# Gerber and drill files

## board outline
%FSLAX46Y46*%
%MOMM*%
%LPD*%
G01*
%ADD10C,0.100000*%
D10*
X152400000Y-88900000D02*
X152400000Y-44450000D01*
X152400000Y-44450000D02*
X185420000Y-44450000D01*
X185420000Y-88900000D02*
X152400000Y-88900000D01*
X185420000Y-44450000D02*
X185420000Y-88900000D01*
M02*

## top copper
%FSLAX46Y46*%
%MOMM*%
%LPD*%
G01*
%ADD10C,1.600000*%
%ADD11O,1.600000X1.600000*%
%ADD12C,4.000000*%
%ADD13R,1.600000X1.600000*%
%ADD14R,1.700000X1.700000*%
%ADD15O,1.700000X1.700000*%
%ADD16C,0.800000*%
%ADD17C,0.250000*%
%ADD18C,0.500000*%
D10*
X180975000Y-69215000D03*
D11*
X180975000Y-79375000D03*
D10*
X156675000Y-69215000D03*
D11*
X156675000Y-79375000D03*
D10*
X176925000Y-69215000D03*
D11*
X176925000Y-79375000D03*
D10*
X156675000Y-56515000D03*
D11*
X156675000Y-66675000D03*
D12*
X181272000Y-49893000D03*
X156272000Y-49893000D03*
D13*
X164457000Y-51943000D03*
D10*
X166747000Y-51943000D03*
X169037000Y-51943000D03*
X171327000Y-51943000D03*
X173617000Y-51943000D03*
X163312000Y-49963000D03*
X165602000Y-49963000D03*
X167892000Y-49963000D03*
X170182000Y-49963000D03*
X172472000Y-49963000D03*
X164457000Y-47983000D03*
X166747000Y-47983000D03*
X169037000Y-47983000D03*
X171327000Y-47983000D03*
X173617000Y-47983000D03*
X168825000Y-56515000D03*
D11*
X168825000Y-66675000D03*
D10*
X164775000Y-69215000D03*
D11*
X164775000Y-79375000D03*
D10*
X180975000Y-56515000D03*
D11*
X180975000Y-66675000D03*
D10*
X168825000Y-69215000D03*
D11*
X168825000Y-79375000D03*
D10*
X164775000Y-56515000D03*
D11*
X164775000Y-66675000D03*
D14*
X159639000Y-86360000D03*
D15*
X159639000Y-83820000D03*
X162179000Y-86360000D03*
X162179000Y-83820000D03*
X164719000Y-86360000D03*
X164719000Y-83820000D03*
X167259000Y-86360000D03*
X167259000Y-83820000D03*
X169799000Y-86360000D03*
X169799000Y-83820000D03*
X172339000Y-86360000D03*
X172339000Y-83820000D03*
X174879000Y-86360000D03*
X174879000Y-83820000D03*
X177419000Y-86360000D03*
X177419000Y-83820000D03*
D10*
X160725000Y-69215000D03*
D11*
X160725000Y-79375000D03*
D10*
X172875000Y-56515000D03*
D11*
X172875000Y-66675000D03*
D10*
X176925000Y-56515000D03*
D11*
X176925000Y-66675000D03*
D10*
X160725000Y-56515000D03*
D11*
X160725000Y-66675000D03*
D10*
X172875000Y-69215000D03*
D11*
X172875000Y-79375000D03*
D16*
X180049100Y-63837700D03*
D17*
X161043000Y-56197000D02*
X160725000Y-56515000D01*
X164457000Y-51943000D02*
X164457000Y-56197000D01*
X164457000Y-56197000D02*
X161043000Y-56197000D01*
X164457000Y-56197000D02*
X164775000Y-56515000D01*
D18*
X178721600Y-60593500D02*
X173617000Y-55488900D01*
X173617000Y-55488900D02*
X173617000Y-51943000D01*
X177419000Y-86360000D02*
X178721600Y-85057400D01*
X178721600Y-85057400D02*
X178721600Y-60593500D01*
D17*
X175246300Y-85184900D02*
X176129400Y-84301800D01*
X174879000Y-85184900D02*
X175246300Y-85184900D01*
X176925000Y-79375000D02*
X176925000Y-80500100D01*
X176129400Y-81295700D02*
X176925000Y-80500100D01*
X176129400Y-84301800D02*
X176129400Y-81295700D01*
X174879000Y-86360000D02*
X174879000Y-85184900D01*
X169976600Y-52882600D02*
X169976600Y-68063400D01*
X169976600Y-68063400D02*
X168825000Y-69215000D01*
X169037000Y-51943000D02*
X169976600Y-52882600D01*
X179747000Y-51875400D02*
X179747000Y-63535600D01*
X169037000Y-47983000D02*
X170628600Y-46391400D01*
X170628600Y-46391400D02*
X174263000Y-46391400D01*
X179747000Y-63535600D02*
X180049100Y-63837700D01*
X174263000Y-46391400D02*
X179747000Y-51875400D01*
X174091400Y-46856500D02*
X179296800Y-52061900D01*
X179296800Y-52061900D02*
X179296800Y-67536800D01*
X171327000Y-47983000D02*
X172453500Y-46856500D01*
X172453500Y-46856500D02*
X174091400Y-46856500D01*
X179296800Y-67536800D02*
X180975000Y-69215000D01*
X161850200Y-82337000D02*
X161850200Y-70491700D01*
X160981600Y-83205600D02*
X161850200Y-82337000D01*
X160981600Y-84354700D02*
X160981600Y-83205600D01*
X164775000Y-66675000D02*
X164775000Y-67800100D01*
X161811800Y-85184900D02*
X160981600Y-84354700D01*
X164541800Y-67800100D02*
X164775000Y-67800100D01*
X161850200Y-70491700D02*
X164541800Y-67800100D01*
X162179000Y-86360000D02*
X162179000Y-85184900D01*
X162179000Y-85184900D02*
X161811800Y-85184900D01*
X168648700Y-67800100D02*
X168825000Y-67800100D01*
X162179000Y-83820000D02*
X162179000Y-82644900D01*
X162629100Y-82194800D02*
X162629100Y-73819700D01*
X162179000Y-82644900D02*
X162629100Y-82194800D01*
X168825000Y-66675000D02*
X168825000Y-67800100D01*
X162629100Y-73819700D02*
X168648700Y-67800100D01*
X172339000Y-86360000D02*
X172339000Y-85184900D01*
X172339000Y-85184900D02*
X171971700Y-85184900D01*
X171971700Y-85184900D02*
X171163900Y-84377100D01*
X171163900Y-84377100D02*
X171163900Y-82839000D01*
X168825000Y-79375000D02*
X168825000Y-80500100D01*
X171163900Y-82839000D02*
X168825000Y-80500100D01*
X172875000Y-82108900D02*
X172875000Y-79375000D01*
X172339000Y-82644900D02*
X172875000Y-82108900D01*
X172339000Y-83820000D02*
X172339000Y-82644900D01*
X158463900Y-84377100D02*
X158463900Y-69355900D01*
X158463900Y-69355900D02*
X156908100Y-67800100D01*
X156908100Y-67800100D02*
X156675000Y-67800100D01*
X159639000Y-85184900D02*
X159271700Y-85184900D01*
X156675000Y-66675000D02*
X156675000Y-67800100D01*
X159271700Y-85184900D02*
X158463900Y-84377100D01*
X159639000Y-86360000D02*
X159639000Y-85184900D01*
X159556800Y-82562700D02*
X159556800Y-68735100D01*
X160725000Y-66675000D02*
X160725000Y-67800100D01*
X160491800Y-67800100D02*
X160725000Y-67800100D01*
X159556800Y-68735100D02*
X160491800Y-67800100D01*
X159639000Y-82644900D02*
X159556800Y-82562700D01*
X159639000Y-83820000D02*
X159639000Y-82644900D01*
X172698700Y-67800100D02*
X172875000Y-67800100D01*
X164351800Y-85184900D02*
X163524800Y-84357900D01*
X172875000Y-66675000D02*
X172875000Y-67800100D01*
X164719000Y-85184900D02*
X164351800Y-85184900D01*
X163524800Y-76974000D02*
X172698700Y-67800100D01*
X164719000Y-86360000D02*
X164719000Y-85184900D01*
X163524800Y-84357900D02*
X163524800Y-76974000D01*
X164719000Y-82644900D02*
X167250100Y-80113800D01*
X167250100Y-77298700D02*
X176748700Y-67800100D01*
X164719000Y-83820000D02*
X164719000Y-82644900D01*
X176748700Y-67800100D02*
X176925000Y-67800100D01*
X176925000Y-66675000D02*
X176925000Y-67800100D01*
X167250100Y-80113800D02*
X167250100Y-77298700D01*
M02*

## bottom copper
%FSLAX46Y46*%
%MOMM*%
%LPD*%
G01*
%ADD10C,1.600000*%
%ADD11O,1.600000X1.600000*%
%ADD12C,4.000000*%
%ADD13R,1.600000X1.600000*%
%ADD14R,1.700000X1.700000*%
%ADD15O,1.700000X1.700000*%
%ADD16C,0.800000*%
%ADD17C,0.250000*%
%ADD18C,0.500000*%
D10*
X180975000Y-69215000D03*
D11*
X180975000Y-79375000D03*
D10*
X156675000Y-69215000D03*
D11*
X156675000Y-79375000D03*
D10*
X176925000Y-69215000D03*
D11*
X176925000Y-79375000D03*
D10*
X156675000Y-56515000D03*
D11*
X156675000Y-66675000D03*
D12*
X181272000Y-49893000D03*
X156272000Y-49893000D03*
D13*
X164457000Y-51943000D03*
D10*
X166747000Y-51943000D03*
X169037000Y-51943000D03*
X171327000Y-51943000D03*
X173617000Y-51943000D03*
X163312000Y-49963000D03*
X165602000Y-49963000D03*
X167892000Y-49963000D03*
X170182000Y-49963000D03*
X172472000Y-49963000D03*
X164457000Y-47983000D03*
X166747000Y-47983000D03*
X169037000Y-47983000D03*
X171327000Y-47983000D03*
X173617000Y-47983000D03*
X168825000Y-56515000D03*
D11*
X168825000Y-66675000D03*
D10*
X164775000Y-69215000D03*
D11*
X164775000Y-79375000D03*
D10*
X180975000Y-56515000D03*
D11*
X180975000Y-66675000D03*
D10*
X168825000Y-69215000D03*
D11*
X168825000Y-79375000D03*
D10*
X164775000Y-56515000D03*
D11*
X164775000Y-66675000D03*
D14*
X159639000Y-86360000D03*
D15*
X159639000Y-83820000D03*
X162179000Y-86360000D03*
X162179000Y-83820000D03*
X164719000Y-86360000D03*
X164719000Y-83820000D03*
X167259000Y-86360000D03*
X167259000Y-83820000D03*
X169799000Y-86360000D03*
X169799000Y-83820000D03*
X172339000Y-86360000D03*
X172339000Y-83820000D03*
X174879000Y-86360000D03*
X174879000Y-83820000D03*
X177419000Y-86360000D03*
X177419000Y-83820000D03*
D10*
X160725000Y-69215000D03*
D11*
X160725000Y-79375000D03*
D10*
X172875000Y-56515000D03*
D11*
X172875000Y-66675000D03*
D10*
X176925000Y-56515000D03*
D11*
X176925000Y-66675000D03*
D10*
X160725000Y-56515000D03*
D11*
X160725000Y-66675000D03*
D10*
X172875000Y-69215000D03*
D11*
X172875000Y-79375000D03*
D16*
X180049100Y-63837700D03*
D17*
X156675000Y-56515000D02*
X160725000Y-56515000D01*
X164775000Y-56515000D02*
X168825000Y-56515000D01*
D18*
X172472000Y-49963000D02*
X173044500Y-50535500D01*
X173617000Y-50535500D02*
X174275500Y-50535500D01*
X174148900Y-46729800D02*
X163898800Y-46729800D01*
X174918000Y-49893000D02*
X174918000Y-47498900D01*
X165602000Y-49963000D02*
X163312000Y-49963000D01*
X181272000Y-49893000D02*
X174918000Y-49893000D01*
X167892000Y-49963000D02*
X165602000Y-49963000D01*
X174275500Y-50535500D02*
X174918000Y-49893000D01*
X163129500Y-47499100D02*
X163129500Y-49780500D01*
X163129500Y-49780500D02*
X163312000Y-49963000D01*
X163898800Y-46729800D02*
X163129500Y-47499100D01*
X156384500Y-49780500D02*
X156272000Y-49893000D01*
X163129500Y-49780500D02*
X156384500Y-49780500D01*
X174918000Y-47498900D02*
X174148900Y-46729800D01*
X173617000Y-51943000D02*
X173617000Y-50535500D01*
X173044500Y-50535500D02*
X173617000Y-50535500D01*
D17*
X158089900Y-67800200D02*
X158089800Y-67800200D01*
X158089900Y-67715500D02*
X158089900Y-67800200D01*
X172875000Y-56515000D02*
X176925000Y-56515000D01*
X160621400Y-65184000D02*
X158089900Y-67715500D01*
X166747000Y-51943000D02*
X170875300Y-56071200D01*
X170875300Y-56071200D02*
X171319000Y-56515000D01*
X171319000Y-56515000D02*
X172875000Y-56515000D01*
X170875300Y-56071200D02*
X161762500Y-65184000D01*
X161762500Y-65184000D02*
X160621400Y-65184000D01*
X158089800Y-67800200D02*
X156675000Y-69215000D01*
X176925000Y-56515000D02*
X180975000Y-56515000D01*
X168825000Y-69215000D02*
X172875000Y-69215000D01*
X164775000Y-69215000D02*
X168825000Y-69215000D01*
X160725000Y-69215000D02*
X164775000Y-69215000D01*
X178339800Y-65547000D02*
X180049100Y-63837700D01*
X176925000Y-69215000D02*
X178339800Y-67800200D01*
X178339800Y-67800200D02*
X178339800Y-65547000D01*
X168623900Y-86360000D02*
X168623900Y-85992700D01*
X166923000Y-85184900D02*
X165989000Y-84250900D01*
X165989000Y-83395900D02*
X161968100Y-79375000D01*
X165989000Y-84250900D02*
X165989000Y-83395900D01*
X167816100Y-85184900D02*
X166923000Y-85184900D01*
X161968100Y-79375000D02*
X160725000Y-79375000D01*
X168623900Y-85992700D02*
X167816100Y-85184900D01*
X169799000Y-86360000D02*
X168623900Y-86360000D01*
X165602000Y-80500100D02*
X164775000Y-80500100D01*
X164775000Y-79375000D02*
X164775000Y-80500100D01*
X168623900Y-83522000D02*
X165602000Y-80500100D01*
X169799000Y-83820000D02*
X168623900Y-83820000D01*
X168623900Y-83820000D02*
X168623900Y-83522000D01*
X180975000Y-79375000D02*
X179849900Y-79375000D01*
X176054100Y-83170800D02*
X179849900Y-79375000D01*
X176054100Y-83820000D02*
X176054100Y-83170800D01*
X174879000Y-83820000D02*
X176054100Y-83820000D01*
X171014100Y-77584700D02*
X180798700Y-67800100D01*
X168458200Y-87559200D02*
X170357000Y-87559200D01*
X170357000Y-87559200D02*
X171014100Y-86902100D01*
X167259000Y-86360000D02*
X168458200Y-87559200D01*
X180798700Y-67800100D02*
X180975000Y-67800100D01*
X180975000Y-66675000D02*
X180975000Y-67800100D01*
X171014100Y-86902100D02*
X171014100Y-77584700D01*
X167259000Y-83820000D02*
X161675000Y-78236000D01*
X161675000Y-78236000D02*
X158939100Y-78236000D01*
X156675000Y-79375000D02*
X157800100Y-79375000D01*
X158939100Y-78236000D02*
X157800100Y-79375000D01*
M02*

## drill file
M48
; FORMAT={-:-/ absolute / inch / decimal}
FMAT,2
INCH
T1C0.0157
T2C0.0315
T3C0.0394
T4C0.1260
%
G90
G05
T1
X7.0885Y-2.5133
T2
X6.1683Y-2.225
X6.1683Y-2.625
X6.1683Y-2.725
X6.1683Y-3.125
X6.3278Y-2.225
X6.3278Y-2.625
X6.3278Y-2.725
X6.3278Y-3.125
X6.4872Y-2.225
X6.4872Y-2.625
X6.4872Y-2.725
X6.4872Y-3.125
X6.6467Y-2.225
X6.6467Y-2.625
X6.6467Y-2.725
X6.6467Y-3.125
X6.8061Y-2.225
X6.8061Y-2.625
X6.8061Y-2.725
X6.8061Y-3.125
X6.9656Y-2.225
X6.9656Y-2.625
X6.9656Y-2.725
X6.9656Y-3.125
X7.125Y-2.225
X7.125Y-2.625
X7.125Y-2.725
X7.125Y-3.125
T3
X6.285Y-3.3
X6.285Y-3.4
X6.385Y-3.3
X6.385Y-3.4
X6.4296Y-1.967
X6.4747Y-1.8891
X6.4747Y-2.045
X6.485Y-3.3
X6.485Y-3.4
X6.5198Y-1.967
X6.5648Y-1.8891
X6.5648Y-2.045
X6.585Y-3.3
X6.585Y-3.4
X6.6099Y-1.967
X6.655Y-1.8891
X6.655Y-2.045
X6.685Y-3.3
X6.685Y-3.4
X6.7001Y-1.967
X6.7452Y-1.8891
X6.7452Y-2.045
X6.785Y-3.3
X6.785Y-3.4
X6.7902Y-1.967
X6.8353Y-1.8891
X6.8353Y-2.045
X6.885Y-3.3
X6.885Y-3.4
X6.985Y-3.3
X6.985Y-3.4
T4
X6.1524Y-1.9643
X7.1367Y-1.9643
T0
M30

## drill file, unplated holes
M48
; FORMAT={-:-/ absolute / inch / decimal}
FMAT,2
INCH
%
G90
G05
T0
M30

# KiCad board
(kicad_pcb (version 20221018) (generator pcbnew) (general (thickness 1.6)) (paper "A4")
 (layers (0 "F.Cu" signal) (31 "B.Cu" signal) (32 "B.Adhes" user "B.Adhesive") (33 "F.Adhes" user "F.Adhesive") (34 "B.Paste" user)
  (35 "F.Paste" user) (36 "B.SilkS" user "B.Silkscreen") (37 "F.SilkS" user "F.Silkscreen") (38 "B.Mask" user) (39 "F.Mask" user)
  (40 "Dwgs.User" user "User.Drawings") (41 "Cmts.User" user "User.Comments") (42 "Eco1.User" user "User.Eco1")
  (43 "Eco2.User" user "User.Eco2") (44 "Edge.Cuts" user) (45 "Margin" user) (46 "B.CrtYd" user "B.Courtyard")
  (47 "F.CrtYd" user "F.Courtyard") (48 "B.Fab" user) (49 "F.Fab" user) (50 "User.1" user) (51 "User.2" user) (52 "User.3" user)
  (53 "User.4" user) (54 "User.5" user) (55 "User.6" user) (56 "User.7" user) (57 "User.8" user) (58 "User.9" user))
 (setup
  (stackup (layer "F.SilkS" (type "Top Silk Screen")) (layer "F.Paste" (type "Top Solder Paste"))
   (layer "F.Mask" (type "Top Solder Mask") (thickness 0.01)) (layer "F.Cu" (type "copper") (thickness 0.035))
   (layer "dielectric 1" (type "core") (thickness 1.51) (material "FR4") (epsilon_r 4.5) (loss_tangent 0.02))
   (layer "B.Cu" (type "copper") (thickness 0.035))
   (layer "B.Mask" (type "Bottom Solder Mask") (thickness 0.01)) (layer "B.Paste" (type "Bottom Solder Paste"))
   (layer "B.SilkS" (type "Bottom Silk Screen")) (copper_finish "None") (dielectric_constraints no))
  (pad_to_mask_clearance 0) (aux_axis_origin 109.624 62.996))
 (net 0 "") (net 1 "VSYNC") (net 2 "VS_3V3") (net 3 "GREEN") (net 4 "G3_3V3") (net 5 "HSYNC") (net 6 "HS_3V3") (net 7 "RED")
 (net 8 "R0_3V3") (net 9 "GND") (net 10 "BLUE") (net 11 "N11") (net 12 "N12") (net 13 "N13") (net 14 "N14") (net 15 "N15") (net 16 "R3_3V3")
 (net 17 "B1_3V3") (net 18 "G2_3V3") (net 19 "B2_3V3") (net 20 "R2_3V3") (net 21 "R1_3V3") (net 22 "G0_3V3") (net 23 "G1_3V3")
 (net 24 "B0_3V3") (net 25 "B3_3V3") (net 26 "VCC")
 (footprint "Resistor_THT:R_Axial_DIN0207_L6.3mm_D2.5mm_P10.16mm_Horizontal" (layer "F.Cu") (at 180.975 69.215 -90)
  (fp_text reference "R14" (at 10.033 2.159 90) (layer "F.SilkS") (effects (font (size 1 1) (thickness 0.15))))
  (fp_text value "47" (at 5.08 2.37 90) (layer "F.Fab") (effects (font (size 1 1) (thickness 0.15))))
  (pad "1" thru_hole circle (at 0 0 270) (size 1.6 1.6) (drill 0.8) (layers "*.Cu" "*.Mask") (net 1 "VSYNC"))
  (pad "2" thru_hole oval (at 10.16 0 270) (size 1.6 1.6) (drill 0.8) (layers "*.Cu" "*.Mask") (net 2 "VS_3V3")))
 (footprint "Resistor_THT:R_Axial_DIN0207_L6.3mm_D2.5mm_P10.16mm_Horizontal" (layer "F.Cu") (at 156.675 69.215 -90)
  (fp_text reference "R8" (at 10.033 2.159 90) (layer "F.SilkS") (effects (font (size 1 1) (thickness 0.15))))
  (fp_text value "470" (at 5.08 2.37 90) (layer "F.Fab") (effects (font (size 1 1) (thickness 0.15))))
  (pad "1" thru_hole circle (at 0 0 270) (size 1.6 1.6) (drill 0.8) (layers "*.Cu" "*.Mask") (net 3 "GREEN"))
  (pad "2" thru_hole oval (at 10.16 0 270) (size 1.6 1.6) (drill 0.8) (layers "*.Cu" "*.Mask") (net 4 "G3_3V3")))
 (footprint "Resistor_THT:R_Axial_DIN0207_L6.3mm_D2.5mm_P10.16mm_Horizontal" (layer "F.Cu") (at 176.925 69.215 -90)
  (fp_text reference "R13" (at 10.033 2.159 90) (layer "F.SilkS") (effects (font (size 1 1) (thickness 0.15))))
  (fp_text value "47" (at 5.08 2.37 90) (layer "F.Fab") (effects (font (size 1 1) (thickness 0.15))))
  (pad "1" thru_hole circle (at 0 0 270) (size 1.6 1.6) (drill 0.8) (layers "*.Cu" "*.Mask") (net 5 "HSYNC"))
  (pad "2" thru_hole oval (at 10.16 0 270) (size 1.6 1.6) (drill 0.8) (layers "*.Cu" "*.Mask") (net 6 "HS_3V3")))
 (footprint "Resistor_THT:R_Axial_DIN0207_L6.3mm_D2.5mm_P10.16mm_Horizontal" (layer "F.Cu") (at 156.675 56.515 -90)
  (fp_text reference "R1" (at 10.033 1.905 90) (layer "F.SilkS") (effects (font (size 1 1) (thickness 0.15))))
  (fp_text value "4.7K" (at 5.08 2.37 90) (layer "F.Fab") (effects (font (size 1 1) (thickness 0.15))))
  (pad "1" thru_hole circle (at 0 0 270) (size 1.6 1.6) (drill 0.8) (layers "*.Cu" "*.Mask") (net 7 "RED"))
  (pad "2" thru_hole oval (at 10.16 0 270) (size 1.6 1.6) (drill 0.8) (layers "*.Cu" "*.Mask") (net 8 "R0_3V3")))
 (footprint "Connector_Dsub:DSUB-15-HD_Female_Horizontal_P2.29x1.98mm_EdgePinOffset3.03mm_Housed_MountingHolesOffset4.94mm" (layer "F.Cu")
  (at 164.457 51.943 180)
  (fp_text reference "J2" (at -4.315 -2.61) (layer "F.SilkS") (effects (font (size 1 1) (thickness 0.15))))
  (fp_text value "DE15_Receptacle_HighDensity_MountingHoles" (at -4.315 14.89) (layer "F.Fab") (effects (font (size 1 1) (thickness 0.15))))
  (pad "0" thru_hole circle (at -16.815 2.05 180) (size 4 4) (drill 3.2) (layers "*.Cu" "*.Mask") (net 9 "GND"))
  (pad "0" thru_hole circle (at 8.185 2.05 180) (size 4 4) (drill 3.2) (layers "*.Cu" "*.Mask") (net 9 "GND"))
  (pad "1" thru_hole rect (at 0 0 180) (size 1.6 1.6) (drill 1) (layers "*.Cu" "*.Mask") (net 7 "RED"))
  (pad "2" thru_hole circle (at -2.29 0 180) (size 1.6 1.6) (drill 1) (layers "*.Cu" "*.Mask") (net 3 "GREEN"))
  (pad "3" thru_hole circle (at -4.58 0 180) (size 1.6 1.6) (drill 1) (layers "*.Cu" "*.Mask") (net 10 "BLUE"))
  (pad "4" thru_hole circle (at -6.87 0 180) (size 1.6 1.6) (drill 1) (layers "*.Cu" "*.Mask") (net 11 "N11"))
  (pad "5" thru_hole circle (at -9.16 0 180) (size 1.6 1.6) (drill 1) (layers "*.Cu" "*.Mask") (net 9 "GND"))
  (pad "6" thru_hole circle (at 1.145 1.98 180) (size 1.6 1.6) (drill 1) (layers "*.Cu" "*.Mask") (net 9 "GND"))
  (pad "7" thru_hole circle (at -1.145 1.98 180) (size 1.6 1.6) (drill 1) (layers "*.Cu" "*.Mask") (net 9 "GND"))
  (pad "8" thru_hole circle (at -3.435 1.98 180) (size 1.6 1.6) (drill 1) (layers "*.Cu" "*.Mask") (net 9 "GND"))
  (pad "9" thru_hole circle (at -5.725 1.98 180) (size 1.6 1.6) (drill 1) (layers "*.Cu" "*.Mask") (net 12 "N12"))
  (pad "10" thru_hole circle (at -8.015 1.98 180) (size 1.6 1.6) (drill 1) (layers "*.Cu" "*.Mask") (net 9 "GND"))
  (pad "11" thru_hole circle (at 0 3.96 180) (size 1.6 1.6) (drill 1) (layers "*.Cu" "*.Mask") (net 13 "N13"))
  (pad "12" thru_hole circle (at -2.29 3.96 180) (size 1.6 1.6) (drill 1) (layers "*.Cu" "*.Mask") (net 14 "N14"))
  (pad "13" thru_hole circle (at -4.58 3.96 180) (size 1.6 1.6) (drill 1) (layers "*.Cu" "*.Mask") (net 5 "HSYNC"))
  (pad "14" thru_hole circle (at -6.87 3.96 180) (size 1.6 1.6) (drill 1) (layers "*.Cu" "*.Mask") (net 1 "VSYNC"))
  (pad "15" thru_hole circle (at -9.16 3.96 180) (size 1.6 1.6) (drill 1) (layers "*.Cu" "*.Mask") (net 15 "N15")))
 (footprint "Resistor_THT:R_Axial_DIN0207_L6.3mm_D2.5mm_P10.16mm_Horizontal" (layer "F.Cu") (at 168.825 56.515 -90)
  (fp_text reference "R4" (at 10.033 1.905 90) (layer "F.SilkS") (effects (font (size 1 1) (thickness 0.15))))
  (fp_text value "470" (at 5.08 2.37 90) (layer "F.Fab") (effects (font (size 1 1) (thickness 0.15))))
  (pad "1" thru_hole circle (at 0 0 270) (size 1.6 1.6) (drill 0.8) (layers "*.Cu" "*.Mask") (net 7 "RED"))
  (pad "2" thru_hole oval (at 10.16 0 270) (size 1.6 1.6) (drill 0.8) (layers "*.Cu" "*.Mask") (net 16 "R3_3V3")))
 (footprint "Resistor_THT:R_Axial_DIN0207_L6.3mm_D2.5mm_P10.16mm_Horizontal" (layer "F.Cu") (at 164.775 69.215 -90)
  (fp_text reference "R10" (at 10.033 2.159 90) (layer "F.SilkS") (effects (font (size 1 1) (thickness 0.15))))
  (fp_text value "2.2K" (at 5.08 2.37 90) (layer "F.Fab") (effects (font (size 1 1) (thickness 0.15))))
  (pad "1" thru_hole circle (at 0 0 270) (size 1.6 1.6) (drill 0.8) (layers "*.Cu" "*.Mask") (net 10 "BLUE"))
  (pad "2" thru_hole oval (at 10.16 0 270) (size 1.6 1.6) (drill 0.8) (layers "*.Cu" "*.Mask") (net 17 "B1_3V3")))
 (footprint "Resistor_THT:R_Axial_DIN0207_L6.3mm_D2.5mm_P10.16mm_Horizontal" (layer "F.Cu") (at 180.975 56.515 -90)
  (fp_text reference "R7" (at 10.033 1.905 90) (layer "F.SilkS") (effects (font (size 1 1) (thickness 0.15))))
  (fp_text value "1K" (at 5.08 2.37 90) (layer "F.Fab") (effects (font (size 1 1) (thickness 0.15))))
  (pad "1" thru_hole circle (at 0 0 270) (size 1.6 1.6) (drill 0.8) (layers "*.Cu" "*.Mask") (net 3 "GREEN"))
  (pad "2" thru_hole oval (at 10.16 0 270) (size 1.6 1.6) (drill 0.8) (layers "*.Cu" "*.Mask") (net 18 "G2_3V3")))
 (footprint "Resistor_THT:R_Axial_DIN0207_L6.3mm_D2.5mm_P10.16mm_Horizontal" (layer "F.Cu") (at 168.825 69.215 -90)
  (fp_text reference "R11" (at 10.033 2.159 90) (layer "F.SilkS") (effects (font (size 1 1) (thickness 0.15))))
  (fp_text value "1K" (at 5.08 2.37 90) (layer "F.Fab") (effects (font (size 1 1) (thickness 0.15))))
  (pad "1" thru_hole circle (at 0 0 270) (size 1.6 1.6) (drill 0.8) (layers "*.Cu" "*.Mask") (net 10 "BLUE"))
  (pad "2" thru_hole oval (at 10.16 0 270) (size 1.6 1.6) (drill 0.8) (layers "*.Cu" "*.Mask") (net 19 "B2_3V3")))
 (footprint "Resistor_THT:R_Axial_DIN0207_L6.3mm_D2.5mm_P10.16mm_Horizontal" (layer "F.Cu") (at 164.775 56.515 -90)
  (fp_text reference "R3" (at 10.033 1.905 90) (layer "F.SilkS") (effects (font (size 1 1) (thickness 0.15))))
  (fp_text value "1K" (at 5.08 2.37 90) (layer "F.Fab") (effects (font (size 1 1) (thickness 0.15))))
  (pad "1" thru_hole circle (at 0 0 270) (size 1.6 1.6) (drill 0.8) (layers "*.Cu" "*.Mask") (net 7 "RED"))
  (pad "2" thru_hole oval (at 10.16 0 270) (size 1.6 1.6) (drill 0.8) (layers "*.Cu" "*.Mask") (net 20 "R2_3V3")))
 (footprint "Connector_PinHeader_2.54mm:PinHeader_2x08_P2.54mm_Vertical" (layer "F.Cu") (at 159.639 86.36 90)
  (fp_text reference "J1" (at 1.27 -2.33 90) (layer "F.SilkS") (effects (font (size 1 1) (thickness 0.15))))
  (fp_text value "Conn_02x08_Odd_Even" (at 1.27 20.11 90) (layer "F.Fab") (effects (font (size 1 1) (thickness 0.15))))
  (pad "1" thru_hole rect (at 0 0 90) (size 1.7 1.7) (drill 1) (layers "*.Cu" "*.Mask") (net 8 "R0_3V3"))
  (pad "2" thru_hole oval (at 2.54 0 90) (size 1.7 1.7) (drill 1) (layers "*.Cu" "*.Mask") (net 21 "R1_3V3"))
  (pad "3" thru_hole oval (at 0 2.54 90) (size 1.7 1.7) (drill 1) (layers "*.Cu" "*.Mask") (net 20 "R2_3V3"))
  (pad "4" thru_hole oval (at 2.54 2.54 90) (size 1.7 1.7) (drill 1) (layers "*.Cu" "*.Mask") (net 16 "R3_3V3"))
  (pad "5" thru_hole oval (at 0 5.08 90) (size 1.7 1.7) (drill 1) (layers "*.Cu" "*.Mask") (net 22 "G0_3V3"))
  (pad "6" thru_hole oval (at 2.54 5.08 90) (size 1.7 1.7) (drill 1) (layers "*.Cu" "*.Mask") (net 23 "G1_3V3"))
  (pad "7" thru_hole oval (at 0 7.62 90) (size 1.7 1.7) (drill 1) (layers "*.Cu" "*.Mask") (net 18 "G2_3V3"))
  (pad "8" thru_hole oval (at 2.54 7.62 90) (size 1.7 1.7) (drill 1) (layers "*.Cu" "*.Mask") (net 4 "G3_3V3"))
  (pad "9" thru_hole oval (at 0 10.16 90) (size 1.7 1.7) (drill 1) (layers "*.Cu" "*.Mask") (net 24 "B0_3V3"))
  (pad "10" thru_hole oval (at 2.54 10.16 90) (size 1.7 1.7) (drill 1) (layers "*.Cu" "*.Mask") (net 17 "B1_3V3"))
  (pad "11" thru_hole oval (at 0 12.7 90) (size 1.7 1.7) (drill 1) (layers "*.Cu" "*.Mask") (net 19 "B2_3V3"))
  (pad "12" thru_hole oval (at 2.54 12.7 90) (size 1.7 1.7) (drill 1) (layers "*.Cu" "*.Mask") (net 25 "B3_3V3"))
  (pad "13" thru_hole oval (at 0 15.24 90) (size 1.7 1.7) (drill 1) (layers "*.Cu" "*.Mask") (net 6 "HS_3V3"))
  (pad "14" thru_hole oval (at 2.54 15.24 90) (size 1.7 1.7) (drill 1) (layers "*.Cu" "*.Mask") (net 2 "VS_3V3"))
  (pad "15" thru_hole oval (at 0 17.78 90) (size 1.7 1.7) (drill 1) (layers "*.Cu" "*.Mask") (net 9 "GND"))
  (pad "16" thru_hole oval (at 2.54 17.78 90) (size 1.7 1.7) (drill 1) (layers "*.Cu" "*.Mask") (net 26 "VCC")))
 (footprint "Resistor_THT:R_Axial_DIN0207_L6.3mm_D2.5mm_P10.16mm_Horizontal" (layer "F.Cu") (at 160.725 69.215 -90)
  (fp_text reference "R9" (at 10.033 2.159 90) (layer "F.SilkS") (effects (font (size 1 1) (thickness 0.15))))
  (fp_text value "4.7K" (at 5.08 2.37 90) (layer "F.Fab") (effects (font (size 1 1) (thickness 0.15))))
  (pad "1" thru_hole circle (at 0 0 270) (size 1.6 1.6) (drill 0.8) (layers "*.Cu" "*.Mask") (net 10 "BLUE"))
  (pad "2" thru_hole oval (at 10.16 0 270) (size 1.6 1.6) (drill 0.8) (layers "*.Cu" "*.Mask") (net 24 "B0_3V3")))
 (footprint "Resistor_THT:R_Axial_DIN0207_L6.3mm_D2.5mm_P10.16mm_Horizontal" (layer "F.Cu") (at 172.875 56.515 -90)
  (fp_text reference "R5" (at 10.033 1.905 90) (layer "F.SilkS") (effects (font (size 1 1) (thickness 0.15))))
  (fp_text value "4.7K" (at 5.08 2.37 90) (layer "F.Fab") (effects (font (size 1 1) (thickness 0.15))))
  (pad "1" thru_hole circle (at 0 0 270) (size 1.6 1.6) (drill 0.8) (layers "*.Cu" "*.Mask") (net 3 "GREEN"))
  (pad "2" thru_hole oval (at 10.16 0 270) (size 1.6 1.6) (drill 0.8) (layers "*.Cu" "*.Mask") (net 22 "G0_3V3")))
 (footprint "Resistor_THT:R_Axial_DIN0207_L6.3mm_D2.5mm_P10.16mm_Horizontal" (layer "F.Cu") (at 176.925 56.515 -90)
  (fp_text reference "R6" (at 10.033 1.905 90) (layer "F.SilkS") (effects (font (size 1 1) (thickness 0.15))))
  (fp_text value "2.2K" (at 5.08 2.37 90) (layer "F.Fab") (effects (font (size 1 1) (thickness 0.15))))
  (pad "1" thru_hole circle (at 0 0 270) (size 1.6 1.6) (drill 0.8) (layers "*.Cu" "*.Mask") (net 3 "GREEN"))
  (pad "2" thru_hole oval (at 10.16 0 270) (size 1.6 1.6) (drill 0.8) (layers "*.Cu" "*.Mask") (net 23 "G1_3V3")))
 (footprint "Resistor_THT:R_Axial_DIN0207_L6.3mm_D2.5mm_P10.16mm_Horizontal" (layer "F.Cu") (at 160.725 56.515 -90)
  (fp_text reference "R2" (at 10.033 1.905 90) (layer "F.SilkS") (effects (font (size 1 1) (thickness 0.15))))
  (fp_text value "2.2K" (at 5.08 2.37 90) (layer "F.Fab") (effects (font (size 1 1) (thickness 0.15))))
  (pad "1" thru_hole circle (at 0 0 270) (size 1.6 1.6) (drill 0.8) (layers "*.Cu" "*.Mask") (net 7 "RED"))
  (pad "2" thru_hole oval (at 10.16 0 270) (size 1.6 1.6) (drill 0.8) (layers "*.Cu" "*.Mask") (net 21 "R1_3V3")))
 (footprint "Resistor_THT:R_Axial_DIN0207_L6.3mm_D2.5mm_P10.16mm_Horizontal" (layer "F.Cu") (at 172.875 69.215 -90)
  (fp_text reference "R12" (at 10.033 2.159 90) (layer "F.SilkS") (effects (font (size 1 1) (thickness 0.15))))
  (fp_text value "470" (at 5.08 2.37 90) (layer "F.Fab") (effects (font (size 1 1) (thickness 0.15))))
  (pad "1" thru_hole circle (at 0 0 270) (size 1.6 1.6) (drill 0.8) (layers "*.Cu" "*.Mask") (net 10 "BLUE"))
  (pad "2" thru_hole oval (at 10.16 0 270) (size 1.6 1.6) (drill 0.8) (layers "*.Cu" "*.Mask") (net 25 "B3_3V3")))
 (gr_line (start 152.4 88.9) (end 152.4 44.45) (stroke (width 0.1) (type default)) (layer "Edge.Cuts"))
 (gr_line (start 152.4 44.45) (end 185.42 44.45) (stroke (width 0.1) (type default)) (layer "Edge.Cuts"))
 (gr_line (start 185.42 88.9) (end 152.4 88.9) (stroke (width 0.1) (type default)) (layer "Edge.Cuts"))
 (gr_line (start 185.42 44.45) (end 185.42 88.9) (stroke (width 0.1) (type default)) (layer "Edge.Cuts"))
 (segment (start 161.043 56.197) (end 160.725 56.515) (width 0.25) (layer "F.Cu") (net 7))
 (segment (start 164.457 51.943) (end 164.457 56.197) (width 0.25) (layer "F.Cu") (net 7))
 (segment (start 164.457 56.197) (end 161.043 56.197) (width 0.25) (layer "F.Cu") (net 7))
 (segment (start 164.457 56.197) (end 164.775 56.515) (width 0.25) (layer "F.Cu") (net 7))
 (segment (start 156.675 56.515) (end 160.725 56.515) (width 0.25) (layer "B.Cu") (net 7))
 (segment (start 164.775 56.515) (end 168.825 56.515) (width 0.25) (layer "B.Cu") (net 7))
 (segment (start 178.7216 60.5935) (end 173.617 55.4889) (width 0.5) (layer "F.Cu") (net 9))
 (segment (start 173.617 55.4889) (end 173.617 51.943) (width 0.5) (layer "F.Cu") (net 9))
 (segment (start 177.419 86.36) (end 178.7216 85.0574) (width 0.5) (layer "F.Cu") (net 9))
 (segment (start 178.7216 85.0574) (end 178.7216 60.5935) (width 0.5) (layer "F.Cu") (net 9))
 (segment (start 172.472 49.963) (end 173.0445 50.5355) (width 0.5) (layer "B.Cu") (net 9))
 (segment (start 173.617 50.5355) (end 174.2755 50.5355) (width 0.5) (layer "B.Cu") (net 9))
 (segment (start 174.1489 46.7298) (end 163.8988 46.7298) (width 0.5) (layer "B.Cu") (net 9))
 (segment (start 174.918 49.893) (end 174.918 47.4989) (width 0.5) (layer "B.Cu") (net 9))
 (segment (start 165.602 49.963) (end 163.312 49.963) (width 0.5) (layer "B.Cu") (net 9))
 (segment (start 181.272 49.893) (end 174.918 49.893) (width 0.5) (layer "B.Cu") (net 9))
 (segment (start 167.892 49.963) (end 165.602 49.963) (width 0.5) (layer "B.Cu") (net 9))
 (segment (start 174.2755 50.5355) (end 174.918 49.893) (width 0.5) (layer "B.Cu") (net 9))
 (segment (start 163.1295 47.4991) (end 163.1295 49.7805) (width 0.5) (layer "B.Cu") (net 9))
 (segment (start 163.1295 49.7805) (end 163.312 49.963) (width 0.5) (layer "B.Cu") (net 9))
 (segment (start 163.8988 46.7298) (end 163.1295 47.4991) (width 0.5) (layer "B.Cu") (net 9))
 (segment (start 156.3845 49.7805) (end 156.272 49.893) (width 0.5) (layer "B.Cu") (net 9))
 (segment (start 163.1295 49.7805) (end 156.3845 49.7805) (width 0.5) (layer "B.Cu") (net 9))
 (segment (start 174.918 47.4989) (end 174.1489 46.7298) (width 0.5) (layer "B.Cu") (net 9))
 (segment (start 173.617 51.943) (end 173.617 50.5355) (width 0.5) (layer "B.Cu") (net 9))
 (segment (start 173.0445 50.5355) (end 173.617 50.5355) (width 0.5) (layer "B.Cu") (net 9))
 (segment (start 180.975 79.375) (end 179.8499 79.375) (width 0.25) (layer "B.Cu") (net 2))
 (segment (start 176.0541 83.1708) (end 179.8499 79.375) (width 0.25) (layer "B.Cu") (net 2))
 (segment (start 176.0541 83.82) (end 176.0541 83.1708) (width 0.25) (layer "B.Cu") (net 2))
 (segment (start 174.879 83.82) (end 176.0541 83.82) (width 0.25) (layer "B.Cu") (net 2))
 (segment (start 158.0899 67.8002) (end 158.0898 67.8002) (width 0.25) (layer "B.Cu") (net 3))
 (segment (start 158.0899 67.7155) (end 158.0899 67.8002) (width 0.25) (layer "B.Cu") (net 3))
 (segment (start 172.875 56.515) (end 176.925 56.515) (width 0.25) (layer "B.Cu") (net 3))
 (segment (start 160.6214 65.184) (end 158.0899 67.7155) (width 0.25) (layer "B.Cu") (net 3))
 (segment (start 166.747 51.943) (end 170.8753 56.0712) (width 0.25) (layer "B.Cu") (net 3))
 (segment (start 170.8753 56.0712) (end 171.319 56.515) (width 0.25) (layer "B.Cu") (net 3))
 (segment (start 171.319 56.515) (end 172.875 56.515) (width 0.25) (layer "B.Cu") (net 3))
 (segment (start 170.8753 56.0712) (end 161.7625 65.184) (width 0.25) (layer "B.Cu") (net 3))
 (segment (start 161.7625 65.184) (end 160.6214 65.184) (width 0.25) (layer "B.Cu") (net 3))
 (segment (start 158.0898 67.8002) (end 156.675 69.215) (width 0.25) (layer "B.Cu") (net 3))
 (segment (start 176.925 56.515) (end 180.975 56.515) (width 0.25) (layer "B.Cu") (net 3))
 (segment (start 169.9766 52.8826) (end 169.9766 68.0634) (width 0.25) (layer "F.Cu") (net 10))
 (segment (start 169.9766 68.0634) (end 168.825 69.215) (width 0.25) (layer "F.Cu") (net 10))
 (segment (start 169.037 51.943) (end 169.9766 52.8826) (width 0.25) (layer "F.Cu") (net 10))
 (segment (start 168.825 69.215) (end 172.875 69.215) (width 0.25) (layer "B.Cu") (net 10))
 (segment (start 164.775 69.215) (end 168.825 69.215) (width 0.25) (layer "B.Cu") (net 10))
 (segment (start 160.725 69.215) (end 164.775 69.215) (width 0.25) (layer "B.Cu") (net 10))
 (segment (start 174.0914 46.8565) (end 179.2968 52.0619) (width 0.25) (layer "F.Cu") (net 1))
 (segment (start 179.2968 52.0619) (end 179.2968 67.5368) (width 0.25) (layer "F.Cu") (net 1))
 (segment (start 171.327 47.983) (end 172.4535 46.8565) (width 0.25) (layer "F.Cu") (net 1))
 (segment (start 172.4535 46.8565) (end 174.0914 46.8565) (width 0.25) (layer "F.Cu") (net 1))
 (segment (start 179.2968 67.5368) (end 180.975 69.215) (width 0.25) (layer "F.Cu") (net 1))
 (segment (start 179.747 51.8754) (end 179.747 63.5356) (width 0.25) (layer "F.Cu") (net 5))
 (segment (start 169.037 47.983) (end 170.6286 46.3914) (width 0.25) (layer "F.Cu") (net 5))
 (segment (start 170.6286 46.3914) (end 174.263 46.3914) (width 0.25) (layer "F.Cu") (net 5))
 (segment (start 179.747 63.5356) (end 180.0491 63.8377) (width 0.25) (layer "F.Cu") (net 5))
 (segment (start 174.263 46.3914) (end 179.747 51.8754) (width 0.25) (layer "F.Cu") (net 5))
 (via (at 180.0491 63.8377) (size 0.8) (drill 0.4) (layers "F.Cu" "B.Cu") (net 5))
 (segment (start 178.3398 65.547) (end 180.0491 63.8377) (width 0.25) (layer "B.Cu") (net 5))
 (segment (start 176.925 69.215) (end 178.3398 67.8002) (width 0.25) (layer "B.Cu") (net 5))
 (segment (start 178.3398 67.8002) (end 178.3398 65.547) (width 0.25) (layer "B.Cu") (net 5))
 (segment (start 161.8502 82.337) (end 161.8502 70.4917) (width 0.25) (layer "F.Cu") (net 20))
 (segment (start 160.9816 83.2056) (end 161.8502 82.337) (width 0.25) (layer "F.Cu") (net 20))
 (segment (start 160.9816 84.3547) (end 160.9816 83.2056) (width 0.25) (layer "F.Cu") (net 20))
 (segment (start 164.775 66.675) (end 164.775 67.8001) (width 0.25) (layer "F.Cu") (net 20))
 (segment (start 161.8118 85.1849) (end 160.9816 84.3547) (width 0.25) (layer "F.Cu") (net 20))
 (segment (start 164.5418 67.8001) (end 164.775 67.8001) (width 0.25) (layer "F.Cu") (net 20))
 (segment (start 161.8502 70.4917) (end 164.5418 67.8001) (width 0.25) (layer "F.Cu") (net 20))
 (segment (start 162.179 86.36) (end 162.179 85.1849) (width 0.25) (layer "F.Cu") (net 20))
 (segment (start 162.179 85.1849) (end 161.8118 85.1849) (width 0.25) (layer "F.Cu") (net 20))
 (segment (start 168.6487 67.8001) (end 168.825 67.8001) (width 0.25) (layer "F.Cu") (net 16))
 (segment (start 162.179 83.82) (end 162.179 82.6449) (width 0.25) (layer "F.Cu") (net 16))
 (segment (start 162.6291 82.1948) (end 162.6291 73.8197) (width 0.25) (layer "F.Cu") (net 16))
 (segment (start 162.179 82.6449) (end 162.6291 82.1948) (width 0.25) (layer "F.Cu") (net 16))
 (segment (start 168.825 66.675) (end 168.825 67.8001) (width 0.25) (layer "F.Cu") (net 16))
 (segment (start 162.6291 73.8197) (end 168.6487 67.8001) (width 0.25) (layer "F.Cu") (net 16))
 (segment (start 168.6239 86.36) (end 168.6239 85.9927) (width 0.25) (layer "B.Cu") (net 24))
 (segment (start 166.923 85.1849) (end 165.989 84.2509) (width 0.25) (layer "B.Cu") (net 24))
 (segment (start 165.989 83.3959) (end 161.9681 79.375) (width 0.25) (layer "B.Cu") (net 24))
 (segment (start 165.989 84.2509) (end 165.989 83.3959) (width 0.25) (layer "B.Cu") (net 24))
 (segment (start 167.8161 85.1849) (end 166.923 85.1849) (width 0.25) (layer "B.Cu") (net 24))
 (segment (start 161.9681 79.375) (end 160.725 79.375) (width 0.25) (layer "B.Cu") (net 24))
 (segment (start 168.6239 85.9927) (end 167.8161 85.1849) (width 0.25) (layer "B.Cu") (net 24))
 (segment (start 169.799 86.36) (end 168.6239 86.36) (width 0.25) (layer "B.Cu") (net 24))
 (segment (start 165.602 80.5001) (end 164.775 80.5001) (width 0.25) (layer "B.Cu") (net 17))
 (segment (start 164.775 79.375) (end 164.775 80.5001) (width 0.25) (layer "B.Cu") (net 17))
 (segment (start 168.6239 83.522) (end 165.602 80.5001) (width 0.25) (layer "B.Cu") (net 17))
 (segment (start 169.799 83.82) (end 168.6239 83.82) (width 0.25) (layer "B.Cu") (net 17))
 (segment (start 168.6239 83.82) (end 168.6239 83.522) (width 0.25) (layer "B.Cu") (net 17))
 (segment (start 172.339 86.36) (end 172.339 85.1849) (width 0.25) (layer "F.Cu") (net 19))
 (segment (start 172.339 85.1849) (end 171.9717 85.1849) (width 0.25) (layer "F.Cu") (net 19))
 (segment (start 171.9717 85.1849) (end 171.1639 84.3771) (width 0.25) (layer "F.Cu") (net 19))
 (segment (start 171.1639 84.3771) (end 171.1639 82.839) (width 0.25) (layer "F.Cu") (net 19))
 (segment (start 168.825 79.375) (end 168.825 80.5001) (width 0.25) (layer "F.Cu") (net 19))
 (segment (start 171.1639 82.839) (end 168.825 80.5001) (width 0.25) (layer "F.Cu") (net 19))
 (segment (start 172.875 82.1089) (end 172.875 79.375) (width 0.25) (layer "F.Cu") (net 25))
 (segment (start 172.339 82.6449) (end 172.875 82.1089) (width 0.25) (layer "F.Cu") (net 25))
 (segment (start 172.339 83.82) (end 172.339 82.6449) (width 0.25) (layer "F.Cu") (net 25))
 (segment (start 175.2463 85.1849) (end 176.1294 84.3018) (width 0.25) (layer "F.Cu") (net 6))
 (segment (start 174.879 85.1849) (end 175.2463 85.1849) (width 0.25) (layer "F.Cu") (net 6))
 (segment (start 176.925 79.375) (end 176.925 80.5001) (width 0.25) (layer "F.Cu") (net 6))
 (segment (start 176.1294 81.2957) (end 176.925 80.5001) (width 0.25) (layer "F.Cu") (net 6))
 (segment (start 176.1294 84.3018) (end 176.1294 81.2957) (width 0.25) (layer "F.Cu") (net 6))
 (segment (start 174.879 86.36) (end 174.879 85.1849) (width 0.25) (layer "F.Cu") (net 6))
 (segment (start 158.4639 84.3771) (end 158.4639 69.3559) (width 0.25) (layer "F.Cu") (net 8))
 (segment (start 158.4639 69.3559) (end 156.9081 67.8001) (width 0.25) (layer "F.Cu") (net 8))
 (segment (start 156.9081 67.8001) (end 156.675 67.8001) (width 0.25) (layer "F.Cu") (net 8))
 (segment (start 159.639 85.1849) (end 159.2717 85.1849) (width 0.25) (layer "F.Cu") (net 8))
 (segment (start 156.675 66.675) (end 156.675 67.8001) (width 0.25) (layer "F.Cu") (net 8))
 (segment (start 159.2717 85.1849) (end 158.4639 84.3771) (width 0.25) (layer "F.Cu") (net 8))
 (segment (start 159.639 86.36) (end 159.639 85.1849) (width 0.25) (layer "F.Cu") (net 8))
 (segment (start 159.5568 82.5627) (end 159.5568 68.7351) (width 0.25) (layer "F.Cu") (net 21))
 (segment (start 160.725 66.675) (end 160.725 67.8001) (width 0.25) (layer "F.Cu") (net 21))
 (segment (start 160.4918 67.8001) (end 160.725 67.8001) (width 0.25) (layer "F.Cu") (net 21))
 (segment (start 159.5568 68.7351) (end 160.4918 67.8001) (width 0.25) (layer "F.Cu") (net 21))
 (segment (start 159.639 82.6449) (end 159.5568 82.5627) (width 0.25) (layer "F.Cu") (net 21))
 (segment (start 159.639 83.82) (end 159.639 82.6449) (width 0.25) (layer "F.Cu") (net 21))
 (segment (start 172.6987 67.8001) (end 172.875 67.8001) (width 0.25) (layer "F.Cu") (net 22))
 (segment (start 164.3518 85.1849) (end 163.5248 84.3579) (width 0.25) (layer "F.Cu") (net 22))
 (segment (start 172.875 66.675) (end 172.875 67.8001) (width 0.25) (layer "F.Cu") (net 22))
 (segment (start 164.719 85.1849) (end 164.3518 85.1849) (width 0.25) (layer "F.Cu") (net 22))
 (segment (start 163.5248 76.974) (end 172.6987 67.8001) (width 0.25) (layer "F.Cu") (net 22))
 (segment (start 164.719 86.36) (end 164.719 85.1849) (width 0.25) (layer "F.Cu") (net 22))
 (segment (start 163.5248 84.3579) (end 163.5248 76.974) (width 0.25) (layer "F.Cu") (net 22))
 (segment (start 164.719 82.6449) (end 167.2501 80.1138) (width 0.25) (layer "F.Cu") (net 23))
 (segment (start 167.2501 77.2987) (end 176.7487 67.8001) (width 0.25) (layer "F.Cu") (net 23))
 (segment (start 164.719 83.82) (end 164.719 82.6449) (width 0.25) (layer "F.Cu") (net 23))
 (segment (start 176.7487 67.8001) (end 176.925 67.8001) (width 0.25) (layer "F.Cu") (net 23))
 (segment (start 176.925 66.675) (end 176.925 67.8001) (width 0.25) (layer "F.Cu") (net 23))
 (segment (start 167.2501 80.1138) (end 167.2501 77.2987) (width 0.25) (layer "F.Cu") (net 23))
 (segment (start 171.0141 77.5847) (end 180.7987 67.8001) (width 0.25) (layer "B.Cu") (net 18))
 (segment (start 168.4582 87.5592) (end 170.357 87.5592) (width 0.25) (layer "B.Cu") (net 18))
 (segment (start 170.357 87.5592) (end 171.0141 86.9021) (width 0.25) (layer "B.Cu") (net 18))
 (segment (start 167.259 86.36) (end 168.4582 87.5592) (width 0.25) (layer "B.Cu") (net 18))
 (segment (start 180.7987 67.8001) (end 180.975 67.8001) (width 0.25) (layer "B.Cu") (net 18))
 (segment (start 180.975 66.675) (end 180.975 67.8001) (width 0.25) (layer "B.Cu") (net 18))
 (segment (start 171.0141 86.9021) (end 171.0141 77.5847) (width 0.25) (layer "B.Cu") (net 18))
 (segment (start 167.259 83.82) (end 161.675 78.236) (width 0.25) (layer "B.Cu") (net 4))
 (segment (start 161.675 78.236) (end 158.9391 78.236) (width 0.25) (layer "B.Cu") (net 4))
 (segment (start 156.675 79.375) (end 157.8001 79.375) (width 0.25) (layer "B.Cu") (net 4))
 (segment (start 158.9391 78.236) (end 157.8001 79.375) (width 0.25) (layer "B.Cu") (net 4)))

